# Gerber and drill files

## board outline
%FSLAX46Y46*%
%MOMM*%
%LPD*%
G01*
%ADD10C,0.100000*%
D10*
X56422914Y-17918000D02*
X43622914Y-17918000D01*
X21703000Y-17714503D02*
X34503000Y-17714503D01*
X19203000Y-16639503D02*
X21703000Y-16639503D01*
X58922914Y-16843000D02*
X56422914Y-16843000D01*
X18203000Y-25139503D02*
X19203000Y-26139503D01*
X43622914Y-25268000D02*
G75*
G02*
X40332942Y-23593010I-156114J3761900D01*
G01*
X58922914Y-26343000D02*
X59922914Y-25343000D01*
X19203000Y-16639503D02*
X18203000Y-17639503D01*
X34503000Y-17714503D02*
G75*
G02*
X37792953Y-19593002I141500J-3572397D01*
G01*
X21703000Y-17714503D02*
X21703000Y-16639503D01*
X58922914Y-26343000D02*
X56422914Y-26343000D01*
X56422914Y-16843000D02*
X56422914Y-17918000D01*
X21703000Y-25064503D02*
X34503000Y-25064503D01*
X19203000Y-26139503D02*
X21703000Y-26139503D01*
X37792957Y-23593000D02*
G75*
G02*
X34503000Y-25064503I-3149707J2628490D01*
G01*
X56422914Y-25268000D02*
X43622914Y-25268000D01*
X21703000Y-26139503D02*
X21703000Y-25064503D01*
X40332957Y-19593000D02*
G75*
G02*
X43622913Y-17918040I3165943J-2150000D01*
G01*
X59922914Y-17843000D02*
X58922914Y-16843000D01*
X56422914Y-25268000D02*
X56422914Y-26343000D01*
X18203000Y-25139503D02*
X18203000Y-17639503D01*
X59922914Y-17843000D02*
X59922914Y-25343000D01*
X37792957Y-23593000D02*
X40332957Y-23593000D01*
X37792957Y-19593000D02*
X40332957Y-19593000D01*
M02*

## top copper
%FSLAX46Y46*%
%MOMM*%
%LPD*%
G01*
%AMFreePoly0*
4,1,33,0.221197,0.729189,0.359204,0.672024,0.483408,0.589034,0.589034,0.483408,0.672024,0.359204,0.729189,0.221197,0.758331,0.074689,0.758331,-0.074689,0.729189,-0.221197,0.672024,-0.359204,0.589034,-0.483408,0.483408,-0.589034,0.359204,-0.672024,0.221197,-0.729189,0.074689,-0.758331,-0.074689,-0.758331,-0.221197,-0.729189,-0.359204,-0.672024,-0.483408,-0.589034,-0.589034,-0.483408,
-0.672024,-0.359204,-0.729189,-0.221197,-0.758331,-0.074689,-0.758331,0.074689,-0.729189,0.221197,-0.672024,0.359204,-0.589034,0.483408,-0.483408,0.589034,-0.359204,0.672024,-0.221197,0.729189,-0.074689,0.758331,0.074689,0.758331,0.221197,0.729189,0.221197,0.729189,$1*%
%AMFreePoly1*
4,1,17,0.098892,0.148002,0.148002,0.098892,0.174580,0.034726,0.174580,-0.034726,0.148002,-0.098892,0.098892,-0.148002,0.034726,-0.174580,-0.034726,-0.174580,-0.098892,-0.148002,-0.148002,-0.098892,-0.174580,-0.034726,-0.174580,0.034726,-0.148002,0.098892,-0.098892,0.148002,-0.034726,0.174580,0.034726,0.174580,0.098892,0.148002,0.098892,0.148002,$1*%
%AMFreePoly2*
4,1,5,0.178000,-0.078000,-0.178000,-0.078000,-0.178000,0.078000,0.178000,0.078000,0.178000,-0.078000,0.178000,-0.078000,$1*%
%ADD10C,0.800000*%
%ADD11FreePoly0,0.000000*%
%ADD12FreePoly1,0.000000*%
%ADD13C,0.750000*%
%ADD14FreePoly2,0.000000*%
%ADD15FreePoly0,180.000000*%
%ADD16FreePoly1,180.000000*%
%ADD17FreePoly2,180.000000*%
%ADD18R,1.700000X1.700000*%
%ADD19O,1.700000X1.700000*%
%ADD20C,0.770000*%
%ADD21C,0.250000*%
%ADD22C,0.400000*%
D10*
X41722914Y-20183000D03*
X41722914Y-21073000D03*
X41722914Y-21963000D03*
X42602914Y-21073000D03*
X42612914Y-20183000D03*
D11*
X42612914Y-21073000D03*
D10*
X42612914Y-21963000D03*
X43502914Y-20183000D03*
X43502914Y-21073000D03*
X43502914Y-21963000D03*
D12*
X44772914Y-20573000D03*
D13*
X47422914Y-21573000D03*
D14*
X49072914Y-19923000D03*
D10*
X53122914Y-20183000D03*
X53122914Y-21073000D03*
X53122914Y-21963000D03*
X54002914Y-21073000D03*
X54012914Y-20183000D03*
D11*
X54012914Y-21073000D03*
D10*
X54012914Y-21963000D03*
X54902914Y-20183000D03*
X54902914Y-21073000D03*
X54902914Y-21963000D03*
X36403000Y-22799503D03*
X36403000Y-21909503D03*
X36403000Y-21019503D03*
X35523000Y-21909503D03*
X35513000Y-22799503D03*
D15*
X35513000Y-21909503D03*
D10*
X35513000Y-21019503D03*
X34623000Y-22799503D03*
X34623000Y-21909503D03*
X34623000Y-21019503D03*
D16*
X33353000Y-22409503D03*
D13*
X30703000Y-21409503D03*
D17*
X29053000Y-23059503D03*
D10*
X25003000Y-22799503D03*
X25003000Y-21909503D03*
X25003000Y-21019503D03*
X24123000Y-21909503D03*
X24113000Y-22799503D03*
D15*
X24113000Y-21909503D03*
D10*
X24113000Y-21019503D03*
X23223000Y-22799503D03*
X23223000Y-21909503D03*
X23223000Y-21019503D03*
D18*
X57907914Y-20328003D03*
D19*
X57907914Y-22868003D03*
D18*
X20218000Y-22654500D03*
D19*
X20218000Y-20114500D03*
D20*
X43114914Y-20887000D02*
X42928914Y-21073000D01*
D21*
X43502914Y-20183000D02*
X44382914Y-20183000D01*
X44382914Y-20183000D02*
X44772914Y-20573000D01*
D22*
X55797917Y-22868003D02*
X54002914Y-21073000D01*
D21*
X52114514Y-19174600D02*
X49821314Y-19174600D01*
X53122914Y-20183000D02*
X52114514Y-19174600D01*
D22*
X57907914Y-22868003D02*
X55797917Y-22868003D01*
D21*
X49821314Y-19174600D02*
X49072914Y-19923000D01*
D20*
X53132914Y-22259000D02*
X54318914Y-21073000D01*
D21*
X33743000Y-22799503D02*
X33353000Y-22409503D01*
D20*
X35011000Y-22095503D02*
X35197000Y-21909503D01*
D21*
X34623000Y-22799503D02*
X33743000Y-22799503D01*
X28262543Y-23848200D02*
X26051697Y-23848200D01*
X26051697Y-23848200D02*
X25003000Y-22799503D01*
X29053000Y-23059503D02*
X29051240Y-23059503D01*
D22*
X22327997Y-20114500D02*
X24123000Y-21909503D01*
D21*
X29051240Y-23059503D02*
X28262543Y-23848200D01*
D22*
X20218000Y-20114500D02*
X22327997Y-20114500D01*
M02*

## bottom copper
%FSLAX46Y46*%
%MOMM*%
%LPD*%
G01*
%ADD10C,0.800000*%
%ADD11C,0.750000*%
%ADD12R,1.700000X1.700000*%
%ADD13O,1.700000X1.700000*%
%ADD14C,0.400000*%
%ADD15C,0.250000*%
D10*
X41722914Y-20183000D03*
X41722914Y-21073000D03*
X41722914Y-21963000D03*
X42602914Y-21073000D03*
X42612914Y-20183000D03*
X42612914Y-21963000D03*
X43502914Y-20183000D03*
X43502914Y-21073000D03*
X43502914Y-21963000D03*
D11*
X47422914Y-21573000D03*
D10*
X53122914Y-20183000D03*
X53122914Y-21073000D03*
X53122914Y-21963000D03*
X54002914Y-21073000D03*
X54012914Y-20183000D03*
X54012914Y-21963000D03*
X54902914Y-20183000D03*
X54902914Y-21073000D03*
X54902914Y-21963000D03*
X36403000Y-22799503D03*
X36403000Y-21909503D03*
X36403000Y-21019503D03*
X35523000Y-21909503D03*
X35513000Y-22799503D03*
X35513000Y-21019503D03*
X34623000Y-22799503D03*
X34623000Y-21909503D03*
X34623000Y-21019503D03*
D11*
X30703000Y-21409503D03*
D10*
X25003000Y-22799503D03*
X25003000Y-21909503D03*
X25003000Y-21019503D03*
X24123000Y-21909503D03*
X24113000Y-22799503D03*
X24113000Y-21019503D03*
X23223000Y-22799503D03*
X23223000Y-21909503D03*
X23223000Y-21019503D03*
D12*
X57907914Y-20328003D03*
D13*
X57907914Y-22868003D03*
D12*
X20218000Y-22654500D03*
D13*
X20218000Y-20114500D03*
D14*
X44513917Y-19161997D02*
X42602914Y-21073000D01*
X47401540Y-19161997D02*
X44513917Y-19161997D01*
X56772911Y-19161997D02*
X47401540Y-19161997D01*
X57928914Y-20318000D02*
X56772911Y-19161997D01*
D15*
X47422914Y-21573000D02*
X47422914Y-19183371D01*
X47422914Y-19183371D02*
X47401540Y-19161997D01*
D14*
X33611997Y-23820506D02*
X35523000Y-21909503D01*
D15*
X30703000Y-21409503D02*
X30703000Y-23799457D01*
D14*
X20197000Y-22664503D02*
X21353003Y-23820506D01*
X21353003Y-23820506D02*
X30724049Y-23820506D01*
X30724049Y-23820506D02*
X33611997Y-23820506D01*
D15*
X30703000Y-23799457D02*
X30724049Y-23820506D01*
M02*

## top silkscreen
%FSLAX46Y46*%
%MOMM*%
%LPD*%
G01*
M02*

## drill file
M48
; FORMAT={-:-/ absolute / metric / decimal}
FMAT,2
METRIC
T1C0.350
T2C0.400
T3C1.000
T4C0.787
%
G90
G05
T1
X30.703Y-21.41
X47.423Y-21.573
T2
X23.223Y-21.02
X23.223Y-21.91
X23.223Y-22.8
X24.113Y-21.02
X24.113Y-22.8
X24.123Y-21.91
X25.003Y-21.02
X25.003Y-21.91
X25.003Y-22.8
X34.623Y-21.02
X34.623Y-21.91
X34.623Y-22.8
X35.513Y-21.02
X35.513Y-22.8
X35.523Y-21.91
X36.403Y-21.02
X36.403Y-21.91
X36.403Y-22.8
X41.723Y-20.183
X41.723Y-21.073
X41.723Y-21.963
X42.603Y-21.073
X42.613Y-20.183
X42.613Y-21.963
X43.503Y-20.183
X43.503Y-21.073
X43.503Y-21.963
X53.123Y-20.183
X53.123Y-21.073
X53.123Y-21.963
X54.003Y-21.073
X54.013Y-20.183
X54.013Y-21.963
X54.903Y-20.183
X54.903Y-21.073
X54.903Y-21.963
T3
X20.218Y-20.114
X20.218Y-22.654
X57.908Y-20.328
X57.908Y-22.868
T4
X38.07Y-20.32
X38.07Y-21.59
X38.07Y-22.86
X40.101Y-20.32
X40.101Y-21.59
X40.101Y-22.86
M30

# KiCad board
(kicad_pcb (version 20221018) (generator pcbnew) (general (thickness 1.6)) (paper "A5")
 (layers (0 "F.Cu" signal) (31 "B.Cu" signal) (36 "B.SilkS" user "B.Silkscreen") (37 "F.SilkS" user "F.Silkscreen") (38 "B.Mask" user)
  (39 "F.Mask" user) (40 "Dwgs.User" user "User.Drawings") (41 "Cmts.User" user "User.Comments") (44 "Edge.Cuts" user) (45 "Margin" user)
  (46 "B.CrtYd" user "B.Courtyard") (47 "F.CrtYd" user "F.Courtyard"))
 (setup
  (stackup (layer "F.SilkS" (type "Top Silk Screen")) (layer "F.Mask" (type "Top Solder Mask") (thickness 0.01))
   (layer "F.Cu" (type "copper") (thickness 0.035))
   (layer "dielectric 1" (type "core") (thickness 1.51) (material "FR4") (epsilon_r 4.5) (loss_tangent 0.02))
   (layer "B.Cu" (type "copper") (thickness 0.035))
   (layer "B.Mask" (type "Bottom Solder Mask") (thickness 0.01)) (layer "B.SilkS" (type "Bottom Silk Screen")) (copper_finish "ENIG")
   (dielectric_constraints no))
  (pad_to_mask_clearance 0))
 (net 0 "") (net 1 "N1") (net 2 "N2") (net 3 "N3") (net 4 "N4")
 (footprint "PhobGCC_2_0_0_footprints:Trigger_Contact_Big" (layer "F.Cu") (at 47.422914 21.573)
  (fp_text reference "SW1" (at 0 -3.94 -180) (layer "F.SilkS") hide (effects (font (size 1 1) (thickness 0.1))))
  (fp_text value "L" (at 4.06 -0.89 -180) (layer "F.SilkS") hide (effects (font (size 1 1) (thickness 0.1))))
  (pad "1" thru_hole circle (at -5.7 -1.39) (size 0.8 0.8) (drill 0.4) (layers "*.Cu" "*.Mask") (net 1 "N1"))
  (pad "1" thru_hole circle (at -5.7 -0.5) (size 0.8 0.8) (drill 0.4) (layers "*.Cu" "*.Mask") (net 1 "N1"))
  (pad "1" thru_hole circle (at -5.7 0.39) (size 0.8 0.8) (drill 0.4) (layers "*.Cu" "*.Mask") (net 1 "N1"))
  (pad "1" thru_hole circle (at -4.82 -0.5) (size 0.8 0.8) (drill 0.4) (layers "*.Cu" "*.Mask") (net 1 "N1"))
  (pad "1" thru_hole circle (at -4.81 -1.39) (size 0.8 0.8) (drill 0.4) (layers "*.Cu" "*.Mask") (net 1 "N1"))
  (pad "1" smd custom (at -4.81 -0.5) (size 1.524 1.524) (layers "F.Cu" "F.Paste" "F.Mask") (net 1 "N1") (thermal_bridge_angle 45)
   (options (clearance outline) (anchor circle)) (primitives))
  (pad "1" thru_hole circle (at -4.81 0.39) (size 0.8 0.8) (drill 0.4) (layers "*.Cu" "*.Mask") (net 1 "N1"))
  (pad "1" thru_hole circle (at -3.92 -1.39) (size 0.8 0.8) (drill 0.4) (layers "*.Cu" "*.Mask") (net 1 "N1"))
  (pad "1" thru_hole circle (at -3.92 -0.5) (size 0.8 0.8) (drill 0.4) (layers "*.Cu" "*.Mask") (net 1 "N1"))
  (pad "1" thru_hole circle (at -3.92 0.39) (size 0.8 0.8) (drill 0.4) (layers "*.Cu" "*.Mask") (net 1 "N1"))
  (pad "1" smd custom (at -2.65 -1) (size 0.356 0.356) (layers "F.Cu" "F.Paste" "F.Mask") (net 1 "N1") (thermal_bridge_angle 45)
   (options (clearance outline) (anchor circle)) (primitives))
  (pad "1" thru_hole circle (at 0 0) (size 0.75 0.75) (drill 0.35) (layers "*.Cu" "*.Mask") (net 1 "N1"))
  (pad "2" smd custom (at 1.65 -1.65) (size 0.356 0.156) (layers "F.Cu" "F.Paste" "F.Mask") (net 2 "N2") (thermal_bridge_angle 45)
   (options (clearance outline) (anchor rect)) (primitives))
  (pad "2" thru_hole circle (at 5.7 -1.39) (size 0.8 0.8) (drill 0.4) (layers "*.Cu" "*.Mask") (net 2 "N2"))
  (pad "2" thru_hole circle (at 5.7 -0.5) (size 0.8 0.8) (drill 0.4) (layers "*.Cu" "*.Mask") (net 2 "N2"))
  (pad "2" thru_hole circle (at 5.7 0.39) (size 0.8 0.8) (drill 0.4) (layers "*.Cu" "*.Mask") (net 2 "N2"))
  (pad "2" thru_hole circle (at 6.58 -0.5) (size 0.8 0.8) (drill 0.4) (layers "*.Cu" "*.Mask") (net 2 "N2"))
  (pad "2" thru_hole circle (at 6.59 -1.39) (size 0.8 0.8) (drill 0.4) (layers "*.Cu" "*.Mask") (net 2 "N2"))
  (pad "2" smd custom (at 6.59 -0.5) (size 1.524 1.524) (layers "F.Cu" "F.Paste" "F.Mask") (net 2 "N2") (thermal_bridge_angle 45)
   (options (clearance outline) (anchor circle)) (primitives))
  (pad "2" thru_hole circle (at 6.59 0.39) (size 0.8 0.8) (drill 0.4) (layers "*.Cu" "*.Mask") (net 2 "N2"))
  (pad "2" thru_hole circle (at 7.48 -1.39) (size 0.8 0.8) (drill 0.4) (layers "*.Cu" "*.Mask") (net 2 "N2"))
  (pad "2" thru_hole circle (at 7.48 -0.5) (size 0.8 0.8) (drill 0.4) (layers "*.Cu" "*.Mask") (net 2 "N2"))
  (pad "2" thru_hole circle (at 7.48 0.39) (size 0.8 0.8) (drill 0.4) (layers "*.Cu" "*.Mask") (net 2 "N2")))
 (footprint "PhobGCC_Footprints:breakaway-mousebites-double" (layer "F.Cu") (at 40.33085 21.36 90)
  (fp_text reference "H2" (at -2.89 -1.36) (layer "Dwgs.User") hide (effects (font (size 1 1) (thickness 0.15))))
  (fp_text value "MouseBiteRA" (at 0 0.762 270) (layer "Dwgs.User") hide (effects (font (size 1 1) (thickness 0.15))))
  (fp_line (start -2.233 -2.537893) (end -2.233 0.002107) (stroke (width 0.1) (type solid)) (layer "Edge.Cuts"))
  (fp_line (start 1.767 -2.537893) (end 1.767 0.002107) (stroke (width 0.1) (type solid)) (layer "Edge.Cuts"))
  (pad "" np_thru_hole circle (at -1.5 -2.26085 270) (size 0.7874 0.7874) (drill 0.7874) (layers "*.Cu" "*.Mask"))
  (pad "" np_thru_hole circle (at -1.5 -0.23 90) (size 0.7874 0.7874) (drill 0.7874) (layers "*.Cu" "*.Mask"))
  (pad "" np_thru_hole circle (at -0.23 -2.26085 270) (size 0.7874 0.7874) (drill 0.7874) (layers "*.Cu" "*.Mask"))
  (pad "" np_thru_hole circle (at -0.23 -0.23 90) (size 0.7874 0.7874) (drill 0.7874) (layers "*.Cu" "*.Mask"))
  (pad "" np_thru_hole circle (at 1.04 -2.26085 270) (size 0.7874 0.7874) (drill 0.7874) (layers "*.Cu" "*.Mask"))
  (pad "" np_thru_hole circle (at 1.04 -0.23 90) (size 0.7874 0.7874) (drill 0.7874) (layers "*.Cu" "*.Mask")))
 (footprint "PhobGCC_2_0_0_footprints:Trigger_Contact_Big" (layer "F.Cu") (at 30.703 21.409503 180)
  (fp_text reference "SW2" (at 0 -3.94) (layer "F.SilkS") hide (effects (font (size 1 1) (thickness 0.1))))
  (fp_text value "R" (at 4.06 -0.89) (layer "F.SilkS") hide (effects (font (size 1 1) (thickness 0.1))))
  (pad "1" thru_hole circle (at -5.7 -1.39 180) (size 0.8 0.8) (drill 0.4) (layers "*.Cu" "*.Mask") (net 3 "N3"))
  (pad "1" thru_hole circle (at -5.7 -0.5 180) (size 0.8 0.8) (drill 0.4) (layers "*.Cu" "*.Mask") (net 3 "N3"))
  (pad "1" thru_hole circle (at -5.7 0.39 180) (size 0.8 0.8) (drill 0.4) (layers "*.Cu" "*.Mask") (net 3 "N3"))
  (pad "1" thru_hole circle (at -4.82 -0.5 180) (size 0.8 0.8) (drill 0.4) (layers "*.Cu" "*.Mask") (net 3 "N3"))
  (pad "1" thru_hole circle (at -4.81 -1.39 180) (size 0.8 0.8) (drill 0.4) (layers "*.Cu" "*.Mask") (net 3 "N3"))
  (pad "1" smd custom (at -4.81 -0.5 180) (size 1.524 1.524) (layers "F.Cu" "F.Paste" "F.Mask") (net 3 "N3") (thermal_bridge_angle 45)
   (options (clearance outline) (anchor circle)) (primitives))
  (pad "1" thru_hole circle (at -4.81 0.39 180) (size 0.8 0.8) (drill 0.4) (layers "*.Cu" "*.Mask") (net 3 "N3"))
  (pad "1" thru_hole circle (at -3.92 -1.39 180) (size 0.8 0.8) (drill 0.4) (layers "*.Cu" "*.Mask") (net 3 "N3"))
  (pad "1" thru_hole circle (at -3.92 -0.5 180) (size 0.8 0.8) (drill 0.4) (layers "*.Cu" "*.Mask") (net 3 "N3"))
  (pad "1" thru_hole circle (at -3.92 0.39 180) (size 0.8 0.8) (drill 0.4) (layers "*.Cu" "*.Mask") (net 3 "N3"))
  (pad "1" smd custom (at -2.65 -1 180) (size 0.356 0.356) (layers "F.Cu" "F.Paste" "F.Mask") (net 3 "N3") (thermal_bridge_angle 45)
   (options (clearance outline) (anchor circle)) (primitives))
  (pad "1" thru_hole circle (at 0 0 180) (size 0.75 0.75) (drill 0.35) (layers "*.Cu" "*.Mask") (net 3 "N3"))
  (pad "2" smd custom (at 1.65 -1.65 180) (size 0.356 0.156) (layers "F.Cu" "F.Paste" "F.Mask") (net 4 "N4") (thermal_bridge_angle 45)
   (options (clearance outline) (anchor rect)) (primitives))
  (pad "2" thru_hole circle (at 5.7 -1.39 180) (size 0.8 0.8) (drill 0.4) (layers "*.Cu" "*.Mask") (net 4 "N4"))
  (pad "2" thru_hole circle (at 5.7 -0.5 180) (size 0.8 0.8) (drill 0.4) (layers "*.Cu" "*.Mask") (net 4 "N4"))
  (pad "2" thru_hole circle (at 5.7 0.39 180) (size 0.8 0.8) (drill 0.4) (layers "*.Cu" "*.Mask") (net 4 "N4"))
  (pad "2" thru_hole circle (at 6.58 -0.5 180) (size 0.8 0.8) (drill 0.4) (layers "*.Cu" "*.Mask") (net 4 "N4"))
  (pad "2" thru_hole circle (at 6.59 -1.39 180) (size 0.8 0.8) (drill 0.4) (layers "*.Cu" "*.Mask") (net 4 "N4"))
  (pad "2" smd custom (at 6.59 -0.5 180) (size 1.524 1.524) (layers "F.Cu" "F.Paste" "F.Mask") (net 4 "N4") (thermal_bridge_angle 45)
   (options (clearance outline) (anchor circle)) (primitives))
  (pad "2" thru_hole circle (at 6.59 0.39 180) (size 0.8 0.8) (drill 0.4) (layers "*.Cu" "*.Mask") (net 4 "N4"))
  (pad "2" thru_hole circle (at 7.48 -1.39 180) (size 0.8 0.8) (drill 0.4) (layers "*.Cu" "*.Mask") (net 4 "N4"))
  (pad "2" thru_hole circle (at 7.48 -0.5 180) (size 0.8 0.8) (drill 0.4) (layers "*.Cu" "*.Mask") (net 4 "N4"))
  (pad "2" thru_hole circle (at 7.48 0.39 180) (size 0.8 0.8) (drill 0.4) (layers "*.Cu" "*.Mask") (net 4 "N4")))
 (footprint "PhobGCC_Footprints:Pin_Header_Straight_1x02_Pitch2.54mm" (layer "B.Cu") (at 57.907914 20.328003 180)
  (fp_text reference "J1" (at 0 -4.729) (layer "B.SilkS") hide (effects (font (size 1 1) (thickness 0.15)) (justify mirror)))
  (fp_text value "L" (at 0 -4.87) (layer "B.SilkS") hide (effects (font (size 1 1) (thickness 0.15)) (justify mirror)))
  (pad "1" thru_hole rect (at 0 0 180) (size 1.7 1.7) (drill 1) (layers "*.Cu" "*.Mask") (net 1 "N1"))
  (pad "2" thru_hole oval (at 0 -2.54 180) (size 1.7 1.7) (drill 1) (layers "*.Cu" "*.Mask") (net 2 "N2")))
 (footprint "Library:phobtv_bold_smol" (layer "B.Cu") (at 49.024943 21.685)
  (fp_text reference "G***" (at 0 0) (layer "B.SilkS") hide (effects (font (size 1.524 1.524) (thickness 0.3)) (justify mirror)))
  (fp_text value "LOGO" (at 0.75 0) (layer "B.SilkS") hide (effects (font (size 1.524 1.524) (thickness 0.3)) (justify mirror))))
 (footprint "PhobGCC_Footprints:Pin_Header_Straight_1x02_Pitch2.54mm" (layer "B.Cu") (at 20.218 22.6545)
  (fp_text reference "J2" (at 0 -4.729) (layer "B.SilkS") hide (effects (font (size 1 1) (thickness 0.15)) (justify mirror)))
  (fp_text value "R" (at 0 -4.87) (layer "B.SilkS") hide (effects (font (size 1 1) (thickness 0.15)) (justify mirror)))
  (pad "1" thru_hole rect (at 0 0) (size 1.7 1.7) (drill 1) (layers "*.Cu" "*.Mask") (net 3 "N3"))
  (pad "2" thru_hole oval (at 0 -2.54) (size 1.7 1.7) (drill 1) (layers "*.Cu" "*.Mask") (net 4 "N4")))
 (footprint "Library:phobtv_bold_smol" (layer "B.Cu") (at 29.124943 21.285 180)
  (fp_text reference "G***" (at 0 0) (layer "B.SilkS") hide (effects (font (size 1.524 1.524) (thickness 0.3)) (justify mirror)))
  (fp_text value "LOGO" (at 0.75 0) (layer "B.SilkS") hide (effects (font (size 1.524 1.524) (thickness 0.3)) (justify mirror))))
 (gr_line (start 56.422914 17.918) (end 43.622914 17.918) (stroke (width 0.1) (type solid)) (layer "Edge.Cuts"))
 (gr_line (start 21.703 17.714503) (end 34.503 17.714503) (stroke (width 0.1) (type solid)) (layer "Edge.Cuts"))
 (gr_line (start 19.203 16.639503) (end 21.703 16.639503) (stroke (width 0.1) (type solid)) (layer "Edge.Cuts"))
 (gr_line (start 58.922914 16.843) (end 56.422914 16.843) (stroke (width 0.1) (type solid)) (layer "Edge.Cuts"))
 (gr_line (start 18.203 25.139503) (end 19.203 26.139503) (stroke (width 0.1) (type solid)) (layer "Edge.Cuts"))
 (gr_arc (start 43.622914 25.268) (mid 41.758548 24.861403) (end 40.332957 23.593) (stroke (width 0.1) (type solid)) (layer "Edge.Cuts"))
 (gr_line (start 58.922914 26.343) (end 59.922914 25.343) (stroke (width 0.1) (type solid)) (layer "Edge.Cuts"))
 (gr_line (start 19.203 16.639503) (end 18.203 17.639503) (stroke (width 0.1) (type solid)) (layer "Edge.Cuts"))
 (gr_arc (start 34.503 17.714503) (mid 36.41725 18.18215) (end 37.792957 19.593) (stroke (width 0.1) (type solid)) (layer "Edge.Cuts"))
 (gr_line (start 21.703 17.714503) (end 21.703 16.639503) (stroke (width 0.1) (type solid)) (layer "Edge.Cuts"))
 (gr_line (start 58.922914 26.343) (end 56.422914 26.343) (stroke (width 0.1) (type solid)) (layer "Edge.Cuts"))
 (gr_line (start 56.422914 16.843) (end 56.422914 17.918) (stroke (width 0.1) (type solid)) (layer "Edge.Cuts"))
 (gr_line (start 21.703 25.064503) (end 34.503 25.064503) (stroke (width 0.1) (type solid)) (layer "Edge.Cuts"))
 (gr_line (start 19.203 26.139503) (end 21.703 26.139503) (stroke (width 0.1) (type solid)) (layer "Edge.Cuts"))
 (gr_arc (start 37.792957 23.593) (mid 36.318224 24.709383) (end 34.503 25.064503) (stroke (width 0.1) (type solid)) (layer "Edge.Cuts"))
 (gr_line (start 56.422914 25.268) (end 43.622914 25.268) (stroke (width 0.1) (type solid)) (layer "Edge.Cuts"))
 (gr_line (start 21.703 26.139503) (end 21.703 25.064503) (stroke (width 0.1) (type solid)) (layer "Edge.Cuts"))
 (gr_arc (start 40.332957 19.593) (mid 41.762608 18.332554) (end 43.622914 17.918) (stroke (width 0.1) (type solid)) (layer "Edge.Cuts"))
 (gr_line (start 59.922914 17.843) (end 58.922914 16.843) (stroke (width 0.1) (type solid)) (layer "Edge.Cuts"))
 (gr_line (start 56.422914 25.268) (end 56.422914 26.343) (stroke (width 0.1) (type solid)) (layer "Edge.Cuts"))
 (gr_line (start 18.203 25.139503) (end 18.203 17.639503) (stroke (width 0.1) (type solid)) (layer "Edge.Cuts"))
 (gr_line (start 59.922914 17.843) (end 59.922914 25.343) (stroke (width 0.1) (type solid)) (layer "Edge.Cuts"))
 (segment (start 43.114914 20.887) (end 42.928914 21.073) (width 0.77) (layer "F.Cu") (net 1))
 (segment (start 43.502914 20.183) (end 44.382914 20.183) (width 0.25) (layer "F.Cu") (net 1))
 (segment (start 44.382914 20.183) (end 44.772914 20.573) (width 0.25) (layer "F.Cu") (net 1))
 (segment (start 44.513917 19.161997) (end 42.602914 21.073) (width 0.4) (layer "B.Cu") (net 1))
 (segment (start 47.40154 19.161997) (end 44.513917 19.161997) (width 0.4) (layer "B.Cu") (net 1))
 (segment (start 56.772911 19.161997) (end 47.40154 19.161997) (width 0.4) (layer "B.Cu") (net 1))
 (segment (start 57.928914 20.318) (end 56.772911 19.161997) (width 0.4) (layer "B.Cu") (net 1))
 (segment (start 47.422914 21.573) (end 47.422914 19.183371) (width 0.25) (layer "B.Cu") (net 1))
 (segment (start 47.422914 19.183371) (end 47.40154 19.161997) (width 0.25) (layer "B.Cu") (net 1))
 (segment (start 55.797917 22.868003) (end 54.002914 21.073) (width 0.4) (layer "F.Cu") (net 2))
 (segment (start 52.114514 19.1746) (end 49.821314 19.1746) (width 0.25) (layer "F.Cu") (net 2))
 (segment (start 53.122914 20.183) (end 52.114514 19.1746) (width 0.25) (layer "F.Cu") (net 2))
 (segment (start 57.907914 22.868003) (end 55.797917 22.868003) (width 0.4) (layer "F.Cu") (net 2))
 (segment (start 49.821314 19.1746) (end 49.072914 19.923) (width 0.25) (layer "F.Cu") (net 2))
 (segment (start 53.132914 22.259) (end 54.318914 21.073) (width 0.77) (layer "F.Cu") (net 2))
 (segment (start 33.743 22.799503) (end 33.353 22.409503) (width 0.25) (layer "F.Cu") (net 3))
 (segment (start 35.011 22.095503) (end 35.197 21.909503) (width 0.77) (layer "F.Cu") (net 3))
 (segment (start 34.623 22.799503) (end 33.743 22.799503) (width 0.25) (layer "F.Cu") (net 3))
 (segment (start 33.611997 23.820506) (end 35.523 21.909503) (width 0.4) (layer "B.Cu") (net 3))
 (segment (start 30.703 21.409503) (end 30.703 23.799457) (width 0.25) (layer "B.Cu") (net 3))
 (segment (start 20.197 22.664503) (end 21.353003 23.820506) (width 0.4) (layer "B.Cu") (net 3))
 (segment (start 21.353003 23.820506) (end 30.724049 23.820506) (width 0.4) (layer "B.Cu") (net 3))
 (segment (start 30.724049 23.820506) (end 33.611997 23.820506) (width 0.4) (layer "B.Cu") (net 3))
 (segment (start 30.703 23.799457) (end 30.724049 23.820506) (width 0.25) (layer "B.Cu") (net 3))
 (segment (start 28.262543 23.8482) (end 26.051697 23.8482) (width 0.25) (layer "F.Cu") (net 4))
 (segment (start 26.051697 23.8482) (end 25.003 22.799503) (width 0.25) (layer "F.Cu") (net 4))
 (segment (start 29.053 23.059503) (end 29.05124 23.059503) (width 0.25) (layer "F.Cu") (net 4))
 (segment (start 22.327997 20.1145) (end 24.123 21.909503) (width 0.4) (layer "F.Cu") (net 4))
 (segment (start 29.05124 23.059503) (end 28.262543 23.8482) (width 0.25) (layer "F.Cu") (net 4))
 (segment (start 20.218 20.1145) (end 22.327997 20.1145) (width 0.4) (layer "F.Cu") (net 4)))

